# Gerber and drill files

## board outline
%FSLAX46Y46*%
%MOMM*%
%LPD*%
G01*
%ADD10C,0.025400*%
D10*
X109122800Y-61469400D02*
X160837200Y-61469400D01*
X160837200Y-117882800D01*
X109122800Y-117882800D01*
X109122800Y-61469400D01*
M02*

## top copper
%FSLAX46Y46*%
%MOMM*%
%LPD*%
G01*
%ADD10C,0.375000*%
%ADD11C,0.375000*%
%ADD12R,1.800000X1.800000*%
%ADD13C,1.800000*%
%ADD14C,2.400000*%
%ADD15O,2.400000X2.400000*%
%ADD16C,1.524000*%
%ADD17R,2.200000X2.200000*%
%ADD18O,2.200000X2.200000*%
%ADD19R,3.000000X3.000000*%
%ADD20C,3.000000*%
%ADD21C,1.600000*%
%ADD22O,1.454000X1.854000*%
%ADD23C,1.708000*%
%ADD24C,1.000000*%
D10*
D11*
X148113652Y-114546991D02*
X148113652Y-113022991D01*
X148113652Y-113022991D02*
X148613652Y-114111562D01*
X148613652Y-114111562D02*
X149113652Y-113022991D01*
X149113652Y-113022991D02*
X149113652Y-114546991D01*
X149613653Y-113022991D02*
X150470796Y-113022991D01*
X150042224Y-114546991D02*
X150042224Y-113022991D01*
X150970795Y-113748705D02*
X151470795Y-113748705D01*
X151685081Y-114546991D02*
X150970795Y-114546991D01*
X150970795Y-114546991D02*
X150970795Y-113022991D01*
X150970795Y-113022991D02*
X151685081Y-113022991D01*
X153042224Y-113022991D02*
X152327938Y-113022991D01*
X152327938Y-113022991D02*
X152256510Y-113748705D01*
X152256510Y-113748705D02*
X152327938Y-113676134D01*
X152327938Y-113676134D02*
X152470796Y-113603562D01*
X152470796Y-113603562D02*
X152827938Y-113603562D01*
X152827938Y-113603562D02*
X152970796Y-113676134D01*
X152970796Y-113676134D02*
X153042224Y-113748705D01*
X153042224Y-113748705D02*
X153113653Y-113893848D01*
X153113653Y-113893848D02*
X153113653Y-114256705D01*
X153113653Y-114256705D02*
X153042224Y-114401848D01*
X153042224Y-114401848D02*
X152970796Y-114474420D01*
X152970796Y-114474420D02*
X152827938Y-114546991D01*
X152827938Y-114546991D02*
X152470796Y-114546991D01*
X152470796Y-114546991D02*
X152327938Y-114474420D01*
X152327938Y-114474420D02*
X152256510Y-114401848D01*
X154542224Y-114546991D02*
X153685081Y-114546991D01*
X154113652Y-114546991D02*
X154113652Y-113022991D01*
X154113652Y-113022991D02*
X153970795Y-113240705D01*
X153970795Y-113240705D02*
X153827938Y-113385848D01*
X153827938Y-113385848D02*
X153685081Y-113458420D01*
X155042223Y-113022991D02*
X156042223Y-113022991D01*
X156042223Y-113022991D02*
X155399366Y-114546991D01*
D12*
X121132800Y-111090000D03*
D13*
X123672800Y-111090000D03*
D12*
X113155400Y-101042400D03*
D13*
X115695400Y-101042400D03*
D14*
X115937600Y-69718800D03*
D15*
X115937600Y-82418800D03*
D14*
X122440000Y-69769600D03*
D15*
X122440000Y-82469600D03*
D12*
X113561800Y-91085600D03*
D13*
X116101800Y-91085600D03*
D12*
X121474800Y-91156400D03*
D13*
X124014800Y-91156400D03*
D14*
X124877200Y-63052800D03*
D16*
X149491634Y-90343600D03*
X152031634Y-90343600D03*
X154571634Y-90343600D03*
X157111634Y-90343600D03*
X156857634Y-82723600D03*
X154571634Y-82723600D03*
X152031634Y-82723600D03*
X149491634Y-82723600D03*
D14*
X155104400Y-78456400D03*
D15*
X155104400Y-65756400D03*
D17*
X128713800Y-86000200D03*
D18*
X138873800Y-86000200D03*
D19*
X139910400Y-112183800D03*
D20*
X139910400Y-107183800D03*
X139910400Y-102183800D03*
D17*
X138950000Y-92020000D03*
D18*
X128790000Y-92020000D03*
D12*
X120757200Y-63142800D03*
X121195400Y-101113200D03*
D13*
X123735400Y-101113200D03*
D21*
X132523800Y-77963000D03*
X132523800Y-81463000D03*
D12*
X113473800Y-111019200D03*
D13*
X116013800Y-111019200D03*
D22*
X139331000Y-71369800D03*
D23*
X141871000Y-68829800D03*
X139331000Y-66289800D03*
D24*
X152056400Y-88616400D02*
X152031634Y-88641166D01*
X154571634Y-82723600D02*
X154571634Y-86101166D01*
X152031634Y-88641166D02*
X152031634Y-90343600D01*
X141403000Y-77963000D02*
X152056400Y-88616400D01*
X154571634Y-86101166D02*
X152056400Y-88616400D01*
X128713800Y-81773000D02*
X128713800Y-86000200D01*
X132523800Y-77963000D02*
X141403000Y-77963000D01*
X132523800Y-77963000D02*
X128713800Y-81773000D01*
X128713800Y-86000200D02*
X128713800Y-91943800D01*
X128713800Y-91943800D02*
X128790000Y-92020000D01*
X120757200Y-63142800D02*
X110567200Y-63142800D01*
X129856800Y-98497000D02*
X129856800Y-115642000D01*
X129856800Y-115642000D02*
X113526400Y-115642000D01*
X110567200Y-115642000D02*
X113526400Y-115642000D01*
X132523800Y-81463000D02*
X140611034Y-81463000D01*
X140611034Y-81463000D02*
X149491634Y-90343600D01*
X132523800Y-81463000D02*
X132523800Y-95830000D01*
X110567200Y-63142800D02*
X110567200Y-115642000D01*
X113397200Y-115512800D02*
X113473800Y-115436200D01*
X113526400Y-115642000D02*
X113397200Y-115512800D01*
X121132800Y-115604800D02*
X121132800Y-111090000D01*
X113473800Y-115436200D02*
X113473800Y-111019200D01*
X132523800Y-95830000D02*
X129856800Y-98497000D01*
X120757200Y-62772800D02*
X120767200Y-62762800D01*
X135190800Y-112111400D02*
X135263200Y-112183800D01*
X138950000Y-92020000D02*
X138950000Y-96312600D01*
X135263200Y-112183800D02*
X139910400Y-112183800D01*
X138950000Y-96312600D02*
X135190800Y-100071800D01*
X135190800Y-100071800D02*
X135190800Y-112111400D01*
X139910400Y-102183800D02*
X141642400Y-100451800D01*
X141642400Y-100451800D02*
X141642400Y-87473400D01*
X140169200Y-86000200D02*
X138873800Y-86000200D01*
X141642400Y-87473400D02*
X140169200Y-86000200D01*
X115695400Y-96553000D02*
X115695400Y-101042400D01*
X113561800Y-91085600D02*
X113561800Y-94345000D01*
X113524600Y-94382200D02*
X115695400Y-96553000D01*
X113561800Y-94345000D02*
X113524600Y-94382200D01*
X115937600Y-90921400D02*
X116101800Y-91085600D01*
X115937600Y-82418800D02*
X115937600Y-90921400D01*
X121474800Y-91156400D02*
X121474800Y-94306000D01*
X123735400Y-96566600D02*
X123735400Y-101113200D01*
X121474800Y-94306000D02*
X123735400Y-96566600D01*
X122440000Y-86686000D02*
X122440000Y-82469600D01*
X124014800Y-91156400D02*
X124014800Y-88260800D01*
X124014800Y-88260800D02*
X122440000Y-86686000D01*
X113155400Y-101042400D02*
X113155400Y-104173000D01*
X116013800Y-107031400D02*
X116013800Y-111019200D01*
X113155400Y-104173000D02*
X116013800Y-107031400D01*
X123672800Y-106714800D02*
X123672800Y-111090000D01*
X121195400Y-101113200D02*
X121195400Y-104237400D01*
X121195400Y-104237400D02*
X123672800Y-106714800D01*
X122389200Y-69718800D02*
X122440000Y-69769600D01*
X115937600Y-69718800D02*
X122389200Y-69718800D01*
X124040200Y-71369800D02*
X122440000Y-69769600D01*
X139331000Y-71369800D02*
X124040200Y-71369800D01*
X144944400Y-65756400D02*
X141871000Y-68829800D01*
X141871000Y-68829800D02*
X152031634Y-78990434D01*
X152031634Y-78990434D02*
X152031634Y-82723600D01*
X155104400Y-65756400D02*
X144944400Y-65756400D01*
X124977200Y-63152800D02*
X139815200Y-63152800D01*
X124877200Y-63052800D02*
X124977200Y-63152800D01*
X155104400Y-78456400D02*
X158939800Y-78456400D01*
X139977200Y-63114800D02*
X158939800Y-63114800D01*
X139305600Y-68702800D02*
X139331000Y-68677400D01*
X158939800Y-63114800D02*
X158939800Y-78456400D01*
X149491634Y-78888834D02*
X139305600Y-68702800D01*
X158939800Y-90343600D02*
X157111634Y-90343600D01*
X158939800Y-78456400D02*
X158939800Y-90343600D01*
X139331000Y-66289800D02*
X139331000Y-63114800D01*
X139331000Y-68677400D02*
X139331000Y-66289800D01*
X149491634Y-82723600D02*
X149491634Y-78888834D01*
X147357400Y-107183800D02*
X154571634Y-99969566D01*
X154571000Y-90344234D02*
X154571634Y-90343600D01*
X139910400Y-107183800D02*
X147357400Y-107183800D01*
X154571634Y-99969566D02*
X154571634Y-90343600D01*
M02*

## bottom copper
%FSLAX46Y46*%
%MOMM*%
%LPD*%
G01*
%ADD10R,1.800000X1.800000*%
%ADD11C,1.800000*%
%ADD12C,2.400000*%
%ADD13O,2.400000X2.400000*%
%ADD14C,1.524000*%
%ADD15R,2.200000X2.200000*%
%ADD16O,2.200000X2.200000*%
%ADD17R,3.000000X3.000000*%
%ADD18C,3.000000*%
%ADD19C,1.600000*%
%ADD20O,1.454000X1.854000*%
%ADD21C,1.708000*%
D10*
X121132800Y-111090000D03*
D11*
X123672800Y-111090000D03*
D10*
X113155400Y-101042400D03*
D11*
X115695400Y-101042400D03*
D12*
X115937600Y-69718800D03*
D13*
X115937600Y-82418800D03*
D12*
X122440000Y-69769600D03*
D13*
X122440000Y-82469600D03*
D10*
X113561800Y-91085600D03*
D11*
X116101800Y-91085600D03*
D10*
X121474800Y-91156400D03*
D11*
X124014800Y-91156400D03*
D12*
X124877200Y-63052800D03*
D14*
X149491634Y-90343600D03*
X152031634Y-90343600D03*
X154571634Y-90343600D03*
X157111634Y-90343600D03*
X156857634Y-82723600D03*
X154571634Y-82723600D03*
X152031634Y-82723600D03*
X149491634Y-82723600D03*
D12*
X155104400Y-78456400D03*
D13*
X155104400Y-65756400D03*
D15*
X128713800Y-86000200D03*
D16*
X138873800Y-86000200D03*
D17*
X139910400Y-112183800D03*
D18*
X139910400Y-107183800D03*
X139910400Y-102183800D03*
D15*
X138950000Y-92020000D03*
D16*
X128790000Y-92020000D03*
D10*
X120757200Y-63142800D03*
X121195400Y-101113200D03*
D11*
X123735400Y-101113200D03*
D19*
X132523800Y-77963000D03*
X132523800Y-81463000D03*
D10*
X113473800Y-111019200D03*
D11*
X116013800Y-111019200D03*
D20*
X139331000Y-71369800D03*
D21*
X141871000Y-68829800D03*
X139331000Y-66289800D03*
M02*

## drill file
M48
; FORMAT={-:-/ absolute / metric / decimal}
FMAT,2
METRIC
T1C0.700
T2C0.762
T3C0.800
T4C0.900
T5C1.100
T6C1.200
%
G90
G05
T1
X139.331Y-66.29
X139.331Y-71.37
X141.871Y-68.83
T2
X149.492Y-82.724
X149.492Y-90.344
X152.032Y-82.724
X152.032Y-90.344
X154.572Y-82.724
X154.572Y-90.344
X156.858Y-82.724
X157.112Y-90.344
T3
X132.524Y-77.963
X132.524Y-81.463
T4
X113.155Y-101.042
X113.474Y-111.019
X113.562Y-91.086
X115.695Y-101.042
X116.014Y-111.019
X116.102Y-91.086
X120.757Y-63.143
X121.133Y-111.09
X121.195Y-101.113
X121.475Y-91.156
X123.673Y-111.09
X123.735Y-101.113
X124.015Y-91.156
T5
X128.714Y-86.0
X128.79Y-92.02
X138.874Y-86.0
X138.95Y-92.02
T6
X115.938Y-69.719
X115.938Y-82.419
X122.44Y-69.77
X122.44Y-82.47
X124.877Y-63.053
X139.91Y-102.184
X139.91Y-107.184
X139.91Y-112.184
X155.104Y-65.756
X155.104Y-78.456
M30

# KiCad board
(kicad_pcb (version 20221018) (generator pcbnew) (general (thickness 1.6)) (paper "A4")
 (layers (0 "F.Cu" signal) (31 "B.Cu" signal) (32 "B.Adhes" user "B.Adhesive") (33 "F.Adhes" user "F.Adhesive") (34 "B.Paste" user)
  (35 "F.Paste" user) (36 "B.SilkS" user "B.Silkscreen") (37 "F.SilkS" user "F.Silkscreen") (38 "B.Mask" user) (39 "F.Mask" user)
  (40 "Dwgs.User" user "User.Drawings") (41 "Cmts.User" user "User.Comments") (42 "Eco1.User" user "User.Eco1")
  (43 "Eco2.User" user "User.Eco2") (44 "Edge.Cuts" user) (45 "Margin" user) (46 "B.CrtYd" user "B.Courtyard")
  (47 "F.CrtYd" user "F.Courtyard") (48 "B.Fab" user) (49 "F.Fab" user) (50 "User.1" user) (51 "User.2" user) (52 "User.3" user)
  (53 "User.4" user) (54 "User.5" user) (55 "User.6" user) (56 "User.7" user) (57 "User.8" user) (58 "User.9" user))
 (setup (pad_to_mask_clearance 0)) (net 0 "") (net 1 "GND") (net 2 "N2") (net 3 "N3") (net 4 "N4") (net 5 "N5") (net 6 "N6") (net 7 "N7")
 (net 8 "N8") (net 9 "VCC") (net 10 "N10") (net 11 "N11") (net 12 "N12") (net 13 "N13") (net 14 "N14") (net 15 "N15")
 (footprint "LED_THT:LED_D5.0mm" (layer "F.Cu") (at 121.1328 111.09)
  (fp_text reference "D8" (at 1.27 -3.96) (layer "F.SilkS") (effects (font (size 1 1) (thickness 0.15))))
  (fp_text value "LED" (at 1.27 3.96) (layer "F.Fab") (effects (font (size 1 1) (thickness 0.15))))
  (pad "1" thru_hole rect (at 0 0) (size 1.8 1.8) (drill 0.9) (layers "*.Cu" "*.Mask") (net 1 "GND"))
  (pad "2" thru_hole circle (at 2.54 0) (size 1.8 1.8) (drill 0.9) (layers "*.Cu" "*.Mask") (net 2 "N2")))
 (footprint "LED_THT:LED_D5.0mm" (layer "F.Cu") (at 113.1554 101.0424)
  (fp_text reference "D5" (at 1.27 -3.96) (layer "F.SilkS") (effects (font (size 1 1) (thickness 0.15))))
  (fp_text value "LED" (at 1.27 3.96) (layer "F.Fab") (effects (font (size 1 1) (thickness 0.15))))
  (pad "1" thru_hole rect (at 0 0) (size 1.8 1.8) (drill 0.9) (layers "*.Cu" "*.Mask") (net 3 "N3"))
  (pad "2" thru_hole circle (at 2.54 0) (size 1.8 1.8) (drill 0.9) (layers "*.Cu" "*.Mask") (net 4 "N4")))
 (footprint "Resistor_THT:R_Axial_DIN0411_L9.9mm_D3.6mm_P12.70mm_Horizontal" (layer "F.Cu") (at 115.9376 69.7188 -90)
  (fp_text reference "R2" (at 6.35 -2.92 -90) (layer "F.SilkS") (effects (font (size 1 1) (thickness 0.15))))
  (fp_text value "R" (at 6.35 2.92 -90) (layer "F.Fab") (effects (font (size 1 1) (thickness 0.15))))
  (pad "1" thru_hole circle (at 0 0 270) (size 2.4 2.4) (drill 1.2) (layers "*.Cu" "*.Mask") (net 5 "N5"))
  (pad "2" thru_hole oval (at 12.7 0 270) (size 2.4 2.4) (drill 1.2) (layers "*.Cu" "*.Mask") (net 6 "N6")))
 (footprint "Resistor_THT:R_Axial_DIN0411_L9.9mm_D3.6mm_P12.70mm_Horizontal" (layer "F.Cu") (at 122.44 69.7696 -90)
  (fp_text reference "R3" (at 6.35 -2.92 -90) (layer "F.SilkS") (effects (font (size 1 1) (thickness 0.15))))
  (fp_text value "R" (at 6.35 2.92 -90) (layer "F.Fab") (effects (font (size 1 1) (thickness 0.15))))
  (pad "1" thru_hole circle (at 0 0 270) (size 2.4 2.4) (drill 1.2) (layers "*.Cu" "*.Mask") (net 5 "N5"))
  (pad "2" thru_hole oval (at 12.7 0 270) (size 2.4 2.4) (drill 1.2) (layers "*.Cu" "*.Mask") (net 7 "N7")))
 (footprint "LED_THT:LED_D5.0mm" (layer "F.Cu") (at 113.5618 91.0856)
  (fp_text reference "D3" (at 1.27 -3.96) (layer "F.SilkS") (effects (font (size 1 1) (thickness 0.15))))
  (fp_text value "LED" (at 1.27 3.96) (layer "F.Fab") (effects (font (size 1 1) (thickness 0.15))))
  (pad "1" thru_hole rect (at 0 0) (size 1.8 1.8) (drill 0.9) (layers "*.Cu" "*.Mask") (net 4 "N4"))
  (pad "2" thru_hole circle (at 2.54 0) (size 1.8 1.8) (drill 0.9) (layers "*.Cu" "*.Mask") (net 6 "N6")))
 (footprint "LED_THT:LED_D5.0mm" (layer "F.Cu") (at 121.4748 91.1564)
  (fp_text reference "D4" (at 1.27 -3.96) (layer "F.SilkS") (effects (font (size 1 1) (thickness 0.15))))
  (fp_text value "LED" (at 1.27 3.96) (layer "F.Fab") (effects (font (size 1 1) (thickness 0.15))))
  (pad "1" thru_hole rect (at 0 0) (size 1.8 1.8) (drill 0.9) (layers "*.Cu" "*.Mask") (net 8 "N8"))
  (pad "2" thru_hole circle (at 2.54 0) (size 1.8 1.8) (drill 0.9) (layers "*.Cu" "*.Mask") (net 7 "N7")))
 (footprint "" (layer "F.Cu") (at 124.8772 63.0528)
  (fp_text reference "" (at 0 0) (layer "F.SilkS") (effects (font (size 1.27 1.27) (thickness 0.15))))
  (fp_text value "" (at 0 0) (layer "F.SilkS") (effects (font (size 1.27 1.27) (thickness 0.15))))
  (pad "1" thru_hole circle (at 0 0 90) (size 2.4 2.4) (drill 1.2) (layers "*.Cu" "*.Mask") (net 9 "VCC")))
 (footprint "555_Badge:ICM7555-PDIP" (layer "F.Cu") (at 153.301634 86.5336)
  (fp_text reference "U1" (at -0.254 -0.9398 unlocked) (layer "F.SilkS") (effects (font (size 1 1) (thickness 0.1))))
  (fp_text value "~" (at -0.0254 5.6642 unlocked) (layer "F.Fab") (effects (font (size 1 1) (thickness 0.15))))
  (pad "1" thru_hole circle (at -3.81 3.81) (size 1.524 1.524) (drill 0.762) (layers "*.Cu" "*.Mask") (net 1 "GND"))
  (pad "2" thru_hole circle (at -1.27 3.81) (size 1.524 1.524) (drill 0.762) (layers "*.Cu" "*.Mask") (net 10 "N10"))
  (pad "3" thru_hole circle (at 1.27 3.81) (size 1.524 1.524) (drill 0.762) (layers "*.Cu" "*.Mask") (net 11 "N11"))
  (pad "4" thru_hole circle (at 3.81 3.81) (size 1.524 1.524) (drill 0.762) (layers "*.Cu" "*.Mask") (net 9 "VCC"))
  (pad "5" thru_hole circle (at 3.556 -3.81) (size 1.524 1.524) (drill 0.762) (layers "*.Cu" "*.Mask") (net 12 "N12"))
  (pad "6" thru_hole circle (at 1.27 -3.81) (size 1.524 1.524) (drill 0.762) (layers "*.Cu" "*.Mask") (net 10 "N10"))
  (pad "7" thru_hole circle (at -1.27 -3.81) (size 1.524 1.524) (drill 0.762) (layers "*.Cu" "*.Mask") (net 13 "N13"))
  (pad "8" thru_hole circle (at -3.81 -3.81) (size 1.524 1.524) (drill 0.762) (layers "*.Cu" "*.Mask") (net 9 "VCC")))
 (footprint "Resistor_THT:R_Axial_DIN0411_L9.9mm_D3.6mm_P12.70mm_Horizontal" (layer "F.Cu") (at 155.1044 78.4564 90)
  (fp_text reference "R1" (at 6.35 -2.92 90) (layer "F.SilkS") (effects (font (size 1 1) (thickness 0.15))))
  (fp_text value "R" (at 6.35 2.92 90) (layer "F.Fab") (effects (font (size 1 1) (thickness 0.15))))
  (pad "1" thru_hole circle (at 0 0 90) (size 2.4 2.4) (drill 1.2) (layers "*.Cu" "*.Mask") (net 9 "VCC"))
  (pad "2" thru_hole oval (at 12.7 0 90) (size 2.4 2.4) (drill 1.2) (layers "*.Cu" "*.Mask") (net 13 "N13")))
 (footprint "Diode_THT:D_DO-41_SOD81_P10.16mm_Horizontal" (layer "F.Cu") (at 128.7138 86.0002)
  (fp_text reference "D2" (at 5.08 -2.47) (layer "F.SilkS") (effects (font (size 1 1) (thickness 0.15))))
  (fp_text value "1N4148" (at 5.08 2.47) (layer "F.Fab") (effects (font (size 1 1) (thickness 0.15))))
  (pad "1" thru_hole rect (at 0 0) (size 2.2 2.2) (drill 1.1) (layers "*.Cu" "*.Mask") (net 10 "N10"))
  (pad "2" thru_hole oval (at 10.16 0) (size 2.2 2.2) (drill 1.1) (layers "*.Cu" "*.Mask") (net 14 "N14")))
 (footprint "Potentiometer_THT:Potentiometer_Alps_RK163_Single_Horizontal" (layer "F.Cu") (at 139.9104 112.1838 180)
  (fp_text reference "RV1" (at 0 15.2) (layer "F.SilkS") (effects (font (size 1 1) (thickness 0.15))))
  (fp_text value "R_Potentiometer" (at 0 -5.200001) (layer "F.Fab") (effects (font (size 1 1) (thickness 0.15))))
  (pad "1" thru_hole rect (at 0 0) (size 3 3) (drill 1.2) (layers "*.Cu" "*.Mask") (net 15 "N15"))
  (pad "2" thru_hole circle (at 0 5) (size 3 3) (drill 1.2) (layers "*.Cu" "*.Mask") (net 11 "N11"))
  (pad "3" thru_hole circle (at 0 10) (size 3 3) (drill 1.2) (layers "*.Cu" "*.Mask") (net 14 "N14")))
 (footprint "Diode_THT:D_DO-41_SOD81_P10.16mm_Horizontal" (layer "F.Cu") (at 138.95 92.02 180)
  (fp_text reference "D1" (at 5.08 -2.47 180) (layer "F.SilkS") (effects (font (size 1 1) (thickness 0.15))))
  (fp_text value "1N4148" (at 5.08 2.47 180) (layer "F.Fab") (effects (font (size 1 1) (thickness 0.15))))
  (pad "1" thru_hole rect (at 0 0 180) (size 2.2 2.2) (drill 1.1) (layers "*.Cu" "*.Mask") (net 15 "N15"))
  (pad "2" thru_hole oval (at 10.16 0 180) (size 2.2 2.2) (drill 1.1) (layers "*.Cu" "*.Mask") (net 10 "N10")))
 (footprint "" (layer "F.Cu") (at 120.7572 63.1428)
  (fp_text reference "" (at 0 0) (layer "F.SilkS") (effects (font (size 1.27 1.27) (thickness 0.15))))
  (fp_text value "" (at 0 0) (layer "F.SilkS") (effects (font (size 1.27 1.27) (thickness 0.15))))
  (pad "1" thru_hole rect (at 0 0) (size 1.8 1.8) (drill 0.9) (layers "*.Cu" "*.Mask") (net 1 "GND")))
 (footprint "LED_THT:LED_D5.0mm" (layer "F.Cu") (at 121.1954 101.1132)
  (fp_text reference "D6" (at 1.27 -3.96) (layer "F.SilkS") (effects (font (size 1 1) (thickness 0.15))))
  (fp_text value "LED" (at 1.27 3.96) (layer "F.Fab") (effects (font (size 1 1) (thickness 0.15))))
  (pad "1" thru_hole rect (at 0 0) (size 1.8 1.8) (drill 0.9) (layers "*.Cu" "*.Mask") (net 2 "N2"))
  (pad "2" thru_hole circle (at 2.54 0) (size 1.8 1.8) (drill 0.9) (layers "*.Cu" "*.Mask") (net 8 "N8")))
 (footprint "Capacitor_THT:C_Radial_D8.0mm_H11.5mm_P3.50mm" (layer "F.Cu") (at 132.5238 77.963 -90)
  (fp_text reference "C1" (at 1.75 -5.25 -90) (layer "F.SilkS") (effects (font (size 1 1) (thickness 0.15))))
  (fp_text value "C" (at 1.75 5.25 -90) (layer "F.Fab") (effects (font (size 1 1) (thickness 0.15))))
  (pad "1" thru_hole circle (at 0 0 270) (size 1.6 1.6) (drill 0.8) (layers "*.Cu" "*.Mask") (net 10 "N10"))
  (pad "2" thru_hole circle (at 3.5 0 270) (size 1.6 1.6) (drill 0.8) (layers "*.Cu" "*.Mask") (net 1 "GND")))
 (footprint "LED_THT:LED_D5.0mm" (layer "F.Cu") (at 113.4738 111.0192)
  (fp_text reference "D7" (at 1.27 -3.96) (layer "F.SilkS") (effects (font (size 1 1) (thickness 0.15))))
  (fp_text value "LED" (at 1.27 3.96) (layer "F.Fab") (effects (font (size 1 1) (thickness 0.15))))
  (pad "1" thru_hole rect (at 0 0) (size 1.8 1.8) (drill 0.9) (layers "*.Cu" "*.Mask") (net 1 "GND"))
  (pad "2" thru_hole circle (at 2.54 0) (size 1.8 1.8) (drill 0.9) (layers "*.Cu" "*.Mask") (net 3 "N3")))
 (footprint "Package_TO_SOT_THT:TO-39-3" (layer "F.Cu") (at 139.331 71.3698 90)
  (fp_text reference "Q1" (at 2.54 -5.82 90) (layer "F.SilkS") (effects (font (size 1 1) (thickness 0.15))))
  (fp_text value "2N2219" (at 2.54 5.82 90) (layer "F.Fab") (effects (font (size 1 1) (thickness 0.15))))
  (pad "1" thru_hole oval (at 0 0 90) (size 1.854 1.454) (drill 0.7) (layers "*.Cu" "*.Mask") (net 5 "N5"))
  (pad "2" thru_hole circle (at 2.54 2.54 90) (size 1.708 1.708) (drill 0.7) (layers "*.Cu" "*.Mask") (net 13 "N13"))
  (pad "3" thru_hole circle (at 5.08 0 90) (size 1.708 1.708) (drill 0.7) (layers "*.Cu" "*.Mask") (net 9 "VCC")))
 (gr_rect (start 109.1228 61.4694) (end 160.8372 117.8828) (stroke (width 0.0254) (type default)) (fill none) (layer "Edge.Cuts"))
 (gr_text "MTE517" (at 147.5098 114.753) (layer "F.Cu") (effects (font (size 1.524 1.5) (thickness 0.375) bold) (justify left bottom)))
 (segment (start 152.0564 88.6164) (end 152.031634 88.641166) (width 1) (layer "F.Cu") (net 10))
 (segment (start 154.571634 82.7236) (end 154.571634 86.101166) (width 1) (layer "F.Cu") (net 10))
 (segment (start 152.031634 88.641166) (end 152.031634 90.3436) (width 1) (layer "F.Cu") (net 10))
 (segment (start 141.403 77.963) (end 152.0564 88.6164) (width 1) (layer "F.Cu") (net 10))
 (segment (start 154.571634 86.101166) (end 152.0564 88.6164) (width 1) (layer "F.Cu") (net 10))
 (segment (start 128.7138 81.773) (end 128.7138 86.0002) (width 1) (layer "F.Cu") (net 10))
 (segment (start 132.5238 77.963) (end 141.403 77.963) (width 1) (layer "F.Cu") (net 10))
 (segment (start 132.5238 77.963) (end 128.7138 81.773) (width 1) (layer "F.Cu") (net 10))
 (segment (start 128.7138 86.0002) (end 128.7138 91.9438) (width 1) (layer "F.Cu") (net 10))
 (segment (start 128.7138 91.9438) (end 128.79 92.02) (width 1) (layer "F.Cu") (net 10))
 (segment (start 120.7572 63.1428) (end 110.5672 63.1428) (width 1) (layer "F.Cu") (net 1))
 (segment (start 129.8568 98.497) (end 129.8568 115.642) (width 1) (layer "F.Cu") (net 1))
 (segment (start 129.8568 115.642) (end 113.5264 115.642) (width 1) (layer "F.Cu") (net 1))
 (segment (start 110.5672 115.642) (end 113.5264 115.642) (width 1) (layer "F.Cu") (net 1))
 (segment (start 132.5238 81.463) (end 140.611034 81.463) (width 1) (layer "F.Cu") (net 1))
 (segment (start 140.611034 81.463) (end 149.491634 90.3436) (width 1) (layer "F.Cu") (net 1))
 (segment (start 132.5238 81.463) (end 132.5238 95.83) (width 1) (layer "F.Cu") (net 1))
 (segment (start 110.5672 63.1428) (end 110.5672 115.642) (width 1) (layer "F.Cu") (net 1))
 (segment (start 113.3972 115.5128) (end 113.4738 115.4362) (width 1) (layer "F.Cu") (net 1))
 (segment (start 113.5264 115.642) (end 113.3972 115.5128) (width 1) (layer "F.Cu") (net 1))
 (segment (start 121.1328 115.6048) (end 121.1328 111.09) (width 1) (layer "F.Cu") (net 1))
 (segment (start 113.4738 115.4362) (end 113.4738 111.0192) (width 1) (layer "F.Cu") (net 1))
 (segment (start 132.5238 95.83) (end 129.8568 98.497) (width 1) (layer "F.Cu") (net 1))
 (segment (start 120.7572 62.7728) (end 120.7672 62.7628) (width 1) (layer "F.Cu") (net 1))
 (segment (start 135.1908 112.1114) (end 135.2632 112.1838) (width 1) (layer "F.Cu") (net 15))
 (segment (start 138.95 92.02) (end 138.95 96.3126) (width 1) (layer "F.Cu") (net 15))
 (segment (start 135.2632 112.1838) (end 139.9104 112.1838) (width 1) (layer "F.Cu") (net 15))
 (segment (start 138.95 96.3126) (end 135.1908 100.0718) (width 1) (layer "F.Cu") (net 15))
 (segment (start 135.1908 100.0718) (end 135.1908 112.1114) (width 1) (layer "F.Cu") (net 15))
 (segment (start 139.9104 102.1838) (end 141.6424 100.4518) (width 1) (layer "F.Cu") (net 14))
 (segment (start 141.6424 100.4518) (end 141.6424 87.4734) (width 1) (layer "F.Cu") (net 14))
 (segment (start 140.1692 86.0002) (end 138.8738 86.0002) (width 1) (layer "F.Cu") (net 14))
 (segment (start 141.6424 87.4734) (end 140.1692 86.0002) (width 1) (layer "F.Cu") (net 14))
 (segment (start 115.6954 96.553) (end 115.6954 101.0424) (width 1) (layer "F.Cu") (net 4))
 (segment (start 113.5618 91.0856) (end 113.5618 94.345) (width 1) (layer "F.Cu") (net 4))
 (segment (start 113.5246 94.3822) (end 115.6954 96.553) (width 1) (layer "F.Cu") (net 4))
 (segment (start 113.5618 94.345) (end 113.5246 94.3822) (width 1) (layer "F.Cu") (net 4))
 (segment (start 115.9376 90.9214) (end 116.1018 91.0856) (width 1) (layer "F.Cu") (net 6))
 (segment (start 115.9376 82.4188) (end 115.9376 90.9214) (width 1) (layer "F.Cu") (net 6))
 (segment (start 121.4748 91.1564) (end 121.4748 94.306) (width 1) (layer "F.Cu") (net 8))
 (segment (start 123.7354 96.5666) (end 123.7354 101.1132) (width 1) (layer "F.Cu") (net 8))
 (segment (start 121.4748 94.306) (end 123.7354 96.5666) (width 1) (layer "F.Cu") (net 8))
 (segment (start 122.44 86.686) (end 122.44 82.4696) (width 1) (layer "F.Cu") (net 7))
 (segment (start 124.0148 91.1564) (end 124.0148 88.2608) (width 1) (layer "F.Cu") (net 7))
 (segment (start 124.0148 88.2608) (end 122.44 86.686) (width 1) (layer "F.Cu") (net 7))
 (segment (start 113.1554 101.0424) (end 113.1554 104.173) (width 1) (layer "F.Cu") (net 3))
 (segment (start 116.0138 107.0314) (end 116.0138 111.0192) (width 1) (layer "F.Cu") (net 3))
 (segment (start 113.1554 104.173) (end 116.0138 107.0314) (width 1) (layer "F.Cu") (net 3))
 (segment (start 123.6728 106.7148) (end 123.6728 111.09) (width 1) (layer "F.Cu") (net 2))
 (segment (start 121.1954 101.1132) (end 121.1954 104.2374) (width 1) (layer "F.Cu") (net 2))
 (segment (start 121.1954 104.2374) (end 123.6728 106.7148) (width 1) (layer "F.Cu") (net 2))
 (segment (start 122.3892 69.7188) (end 122.44 69.7696) (width 1) (layer "F.Cu") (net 5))
 (segment (start 115.9376 69.7188) (end 122.3892 69.7188) (width 1) (layer "F.Cu") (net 5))
 (segment (start 124.0402 71.3698) (end 122.44 69.7696) (width 1) (layer "F.Cu") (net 5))
 (segment (start 139.331 71.3698) (end 124.0402 71.3698) (width 1) (layer "F.Cu") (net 5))
 (segment (start 144.9444 65.7564) (end 141.871 68.8298) (width 1) (layer "F.Cu") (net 13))
 (segment (start 141.871 68.8298) (end 152.031634 78.990434) (width 1) (layer "F.Cu") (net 13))
 (segment (start 152.031634 78.990434) (end 152.031634 82.7236) (width 1) (layer "F.Cu") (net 13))
 (segment (start 155.1044 65.7564) (end 144.9444 65.7564) (width 1) (layer "F.Cu") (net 13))
 (segment (start 124.9772 63.1528) (end 139.8152 63.1528) (width 1) (layer "F.Cu") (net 9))
 (segment (start 124.8772 63.0528) (end 124.9772 63.1528) (width 1) (layer "F.Cu") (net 9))
 (segment (start 155.1044 78.4564) (end 158.9398 78.4564) (width 1) (layer "F.Cu") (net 9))
 (segment (start 139.9772 63.1148) (end 158.9398 63.1148) (width 1) (layer "F.Cu") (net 9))
 (segment (start 139.3056 68.7028) (end 139.331 68.6774) (width 1) (layer "F.Cu") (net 9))
 (segment (start 158.9398 63.1148) (end 158.9398 78.4564) (width 1) (layer "F.Cu") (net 9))
 (segment (start 149.491634 78.888834) (end 139.3056 68.7028) (width 1) (layer "F.Cu") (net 9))
 (segment (start 158.9398 90.3436) (end 157.111634 90.3436) (width 1) (layer "F.Cu") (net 9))
 (segment (start 158.9398 78.4564) (end 158.9398 90.3436) (width 1) (layer "F.Cu") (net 9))
 (segment (start 139.331 66.2898) (end 139.331 63.1148) (width 1) (layer "F.Cu") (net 9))
 (segment (start 139.331 68.6774) (end 139.331 66.2898) (width 1) (layer "F.Cu") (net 9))
 (segment (start 149.491634 82.7236) (end 149.491634 78.888834) (width 1) (layer "F.Cu") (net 9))
 (segment (start 147.3574 107.1838) (end 154.571634 99.969566) (width 1) (layer "F.Cu") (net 11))
 (segment (start 154.571 90.344234) (end 154.571634 90.3436) (width 1) (layer "F.Cu") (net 11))
 (segment (start 139.9104 107.1838) (end 147.3574 107.1838) (width 1) (layer "F.Cu") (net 11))
 (segment (start 154.571634 99.969566) (end 154.571634 90.3436) (width 1) (layer "F.Cu") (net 11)))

